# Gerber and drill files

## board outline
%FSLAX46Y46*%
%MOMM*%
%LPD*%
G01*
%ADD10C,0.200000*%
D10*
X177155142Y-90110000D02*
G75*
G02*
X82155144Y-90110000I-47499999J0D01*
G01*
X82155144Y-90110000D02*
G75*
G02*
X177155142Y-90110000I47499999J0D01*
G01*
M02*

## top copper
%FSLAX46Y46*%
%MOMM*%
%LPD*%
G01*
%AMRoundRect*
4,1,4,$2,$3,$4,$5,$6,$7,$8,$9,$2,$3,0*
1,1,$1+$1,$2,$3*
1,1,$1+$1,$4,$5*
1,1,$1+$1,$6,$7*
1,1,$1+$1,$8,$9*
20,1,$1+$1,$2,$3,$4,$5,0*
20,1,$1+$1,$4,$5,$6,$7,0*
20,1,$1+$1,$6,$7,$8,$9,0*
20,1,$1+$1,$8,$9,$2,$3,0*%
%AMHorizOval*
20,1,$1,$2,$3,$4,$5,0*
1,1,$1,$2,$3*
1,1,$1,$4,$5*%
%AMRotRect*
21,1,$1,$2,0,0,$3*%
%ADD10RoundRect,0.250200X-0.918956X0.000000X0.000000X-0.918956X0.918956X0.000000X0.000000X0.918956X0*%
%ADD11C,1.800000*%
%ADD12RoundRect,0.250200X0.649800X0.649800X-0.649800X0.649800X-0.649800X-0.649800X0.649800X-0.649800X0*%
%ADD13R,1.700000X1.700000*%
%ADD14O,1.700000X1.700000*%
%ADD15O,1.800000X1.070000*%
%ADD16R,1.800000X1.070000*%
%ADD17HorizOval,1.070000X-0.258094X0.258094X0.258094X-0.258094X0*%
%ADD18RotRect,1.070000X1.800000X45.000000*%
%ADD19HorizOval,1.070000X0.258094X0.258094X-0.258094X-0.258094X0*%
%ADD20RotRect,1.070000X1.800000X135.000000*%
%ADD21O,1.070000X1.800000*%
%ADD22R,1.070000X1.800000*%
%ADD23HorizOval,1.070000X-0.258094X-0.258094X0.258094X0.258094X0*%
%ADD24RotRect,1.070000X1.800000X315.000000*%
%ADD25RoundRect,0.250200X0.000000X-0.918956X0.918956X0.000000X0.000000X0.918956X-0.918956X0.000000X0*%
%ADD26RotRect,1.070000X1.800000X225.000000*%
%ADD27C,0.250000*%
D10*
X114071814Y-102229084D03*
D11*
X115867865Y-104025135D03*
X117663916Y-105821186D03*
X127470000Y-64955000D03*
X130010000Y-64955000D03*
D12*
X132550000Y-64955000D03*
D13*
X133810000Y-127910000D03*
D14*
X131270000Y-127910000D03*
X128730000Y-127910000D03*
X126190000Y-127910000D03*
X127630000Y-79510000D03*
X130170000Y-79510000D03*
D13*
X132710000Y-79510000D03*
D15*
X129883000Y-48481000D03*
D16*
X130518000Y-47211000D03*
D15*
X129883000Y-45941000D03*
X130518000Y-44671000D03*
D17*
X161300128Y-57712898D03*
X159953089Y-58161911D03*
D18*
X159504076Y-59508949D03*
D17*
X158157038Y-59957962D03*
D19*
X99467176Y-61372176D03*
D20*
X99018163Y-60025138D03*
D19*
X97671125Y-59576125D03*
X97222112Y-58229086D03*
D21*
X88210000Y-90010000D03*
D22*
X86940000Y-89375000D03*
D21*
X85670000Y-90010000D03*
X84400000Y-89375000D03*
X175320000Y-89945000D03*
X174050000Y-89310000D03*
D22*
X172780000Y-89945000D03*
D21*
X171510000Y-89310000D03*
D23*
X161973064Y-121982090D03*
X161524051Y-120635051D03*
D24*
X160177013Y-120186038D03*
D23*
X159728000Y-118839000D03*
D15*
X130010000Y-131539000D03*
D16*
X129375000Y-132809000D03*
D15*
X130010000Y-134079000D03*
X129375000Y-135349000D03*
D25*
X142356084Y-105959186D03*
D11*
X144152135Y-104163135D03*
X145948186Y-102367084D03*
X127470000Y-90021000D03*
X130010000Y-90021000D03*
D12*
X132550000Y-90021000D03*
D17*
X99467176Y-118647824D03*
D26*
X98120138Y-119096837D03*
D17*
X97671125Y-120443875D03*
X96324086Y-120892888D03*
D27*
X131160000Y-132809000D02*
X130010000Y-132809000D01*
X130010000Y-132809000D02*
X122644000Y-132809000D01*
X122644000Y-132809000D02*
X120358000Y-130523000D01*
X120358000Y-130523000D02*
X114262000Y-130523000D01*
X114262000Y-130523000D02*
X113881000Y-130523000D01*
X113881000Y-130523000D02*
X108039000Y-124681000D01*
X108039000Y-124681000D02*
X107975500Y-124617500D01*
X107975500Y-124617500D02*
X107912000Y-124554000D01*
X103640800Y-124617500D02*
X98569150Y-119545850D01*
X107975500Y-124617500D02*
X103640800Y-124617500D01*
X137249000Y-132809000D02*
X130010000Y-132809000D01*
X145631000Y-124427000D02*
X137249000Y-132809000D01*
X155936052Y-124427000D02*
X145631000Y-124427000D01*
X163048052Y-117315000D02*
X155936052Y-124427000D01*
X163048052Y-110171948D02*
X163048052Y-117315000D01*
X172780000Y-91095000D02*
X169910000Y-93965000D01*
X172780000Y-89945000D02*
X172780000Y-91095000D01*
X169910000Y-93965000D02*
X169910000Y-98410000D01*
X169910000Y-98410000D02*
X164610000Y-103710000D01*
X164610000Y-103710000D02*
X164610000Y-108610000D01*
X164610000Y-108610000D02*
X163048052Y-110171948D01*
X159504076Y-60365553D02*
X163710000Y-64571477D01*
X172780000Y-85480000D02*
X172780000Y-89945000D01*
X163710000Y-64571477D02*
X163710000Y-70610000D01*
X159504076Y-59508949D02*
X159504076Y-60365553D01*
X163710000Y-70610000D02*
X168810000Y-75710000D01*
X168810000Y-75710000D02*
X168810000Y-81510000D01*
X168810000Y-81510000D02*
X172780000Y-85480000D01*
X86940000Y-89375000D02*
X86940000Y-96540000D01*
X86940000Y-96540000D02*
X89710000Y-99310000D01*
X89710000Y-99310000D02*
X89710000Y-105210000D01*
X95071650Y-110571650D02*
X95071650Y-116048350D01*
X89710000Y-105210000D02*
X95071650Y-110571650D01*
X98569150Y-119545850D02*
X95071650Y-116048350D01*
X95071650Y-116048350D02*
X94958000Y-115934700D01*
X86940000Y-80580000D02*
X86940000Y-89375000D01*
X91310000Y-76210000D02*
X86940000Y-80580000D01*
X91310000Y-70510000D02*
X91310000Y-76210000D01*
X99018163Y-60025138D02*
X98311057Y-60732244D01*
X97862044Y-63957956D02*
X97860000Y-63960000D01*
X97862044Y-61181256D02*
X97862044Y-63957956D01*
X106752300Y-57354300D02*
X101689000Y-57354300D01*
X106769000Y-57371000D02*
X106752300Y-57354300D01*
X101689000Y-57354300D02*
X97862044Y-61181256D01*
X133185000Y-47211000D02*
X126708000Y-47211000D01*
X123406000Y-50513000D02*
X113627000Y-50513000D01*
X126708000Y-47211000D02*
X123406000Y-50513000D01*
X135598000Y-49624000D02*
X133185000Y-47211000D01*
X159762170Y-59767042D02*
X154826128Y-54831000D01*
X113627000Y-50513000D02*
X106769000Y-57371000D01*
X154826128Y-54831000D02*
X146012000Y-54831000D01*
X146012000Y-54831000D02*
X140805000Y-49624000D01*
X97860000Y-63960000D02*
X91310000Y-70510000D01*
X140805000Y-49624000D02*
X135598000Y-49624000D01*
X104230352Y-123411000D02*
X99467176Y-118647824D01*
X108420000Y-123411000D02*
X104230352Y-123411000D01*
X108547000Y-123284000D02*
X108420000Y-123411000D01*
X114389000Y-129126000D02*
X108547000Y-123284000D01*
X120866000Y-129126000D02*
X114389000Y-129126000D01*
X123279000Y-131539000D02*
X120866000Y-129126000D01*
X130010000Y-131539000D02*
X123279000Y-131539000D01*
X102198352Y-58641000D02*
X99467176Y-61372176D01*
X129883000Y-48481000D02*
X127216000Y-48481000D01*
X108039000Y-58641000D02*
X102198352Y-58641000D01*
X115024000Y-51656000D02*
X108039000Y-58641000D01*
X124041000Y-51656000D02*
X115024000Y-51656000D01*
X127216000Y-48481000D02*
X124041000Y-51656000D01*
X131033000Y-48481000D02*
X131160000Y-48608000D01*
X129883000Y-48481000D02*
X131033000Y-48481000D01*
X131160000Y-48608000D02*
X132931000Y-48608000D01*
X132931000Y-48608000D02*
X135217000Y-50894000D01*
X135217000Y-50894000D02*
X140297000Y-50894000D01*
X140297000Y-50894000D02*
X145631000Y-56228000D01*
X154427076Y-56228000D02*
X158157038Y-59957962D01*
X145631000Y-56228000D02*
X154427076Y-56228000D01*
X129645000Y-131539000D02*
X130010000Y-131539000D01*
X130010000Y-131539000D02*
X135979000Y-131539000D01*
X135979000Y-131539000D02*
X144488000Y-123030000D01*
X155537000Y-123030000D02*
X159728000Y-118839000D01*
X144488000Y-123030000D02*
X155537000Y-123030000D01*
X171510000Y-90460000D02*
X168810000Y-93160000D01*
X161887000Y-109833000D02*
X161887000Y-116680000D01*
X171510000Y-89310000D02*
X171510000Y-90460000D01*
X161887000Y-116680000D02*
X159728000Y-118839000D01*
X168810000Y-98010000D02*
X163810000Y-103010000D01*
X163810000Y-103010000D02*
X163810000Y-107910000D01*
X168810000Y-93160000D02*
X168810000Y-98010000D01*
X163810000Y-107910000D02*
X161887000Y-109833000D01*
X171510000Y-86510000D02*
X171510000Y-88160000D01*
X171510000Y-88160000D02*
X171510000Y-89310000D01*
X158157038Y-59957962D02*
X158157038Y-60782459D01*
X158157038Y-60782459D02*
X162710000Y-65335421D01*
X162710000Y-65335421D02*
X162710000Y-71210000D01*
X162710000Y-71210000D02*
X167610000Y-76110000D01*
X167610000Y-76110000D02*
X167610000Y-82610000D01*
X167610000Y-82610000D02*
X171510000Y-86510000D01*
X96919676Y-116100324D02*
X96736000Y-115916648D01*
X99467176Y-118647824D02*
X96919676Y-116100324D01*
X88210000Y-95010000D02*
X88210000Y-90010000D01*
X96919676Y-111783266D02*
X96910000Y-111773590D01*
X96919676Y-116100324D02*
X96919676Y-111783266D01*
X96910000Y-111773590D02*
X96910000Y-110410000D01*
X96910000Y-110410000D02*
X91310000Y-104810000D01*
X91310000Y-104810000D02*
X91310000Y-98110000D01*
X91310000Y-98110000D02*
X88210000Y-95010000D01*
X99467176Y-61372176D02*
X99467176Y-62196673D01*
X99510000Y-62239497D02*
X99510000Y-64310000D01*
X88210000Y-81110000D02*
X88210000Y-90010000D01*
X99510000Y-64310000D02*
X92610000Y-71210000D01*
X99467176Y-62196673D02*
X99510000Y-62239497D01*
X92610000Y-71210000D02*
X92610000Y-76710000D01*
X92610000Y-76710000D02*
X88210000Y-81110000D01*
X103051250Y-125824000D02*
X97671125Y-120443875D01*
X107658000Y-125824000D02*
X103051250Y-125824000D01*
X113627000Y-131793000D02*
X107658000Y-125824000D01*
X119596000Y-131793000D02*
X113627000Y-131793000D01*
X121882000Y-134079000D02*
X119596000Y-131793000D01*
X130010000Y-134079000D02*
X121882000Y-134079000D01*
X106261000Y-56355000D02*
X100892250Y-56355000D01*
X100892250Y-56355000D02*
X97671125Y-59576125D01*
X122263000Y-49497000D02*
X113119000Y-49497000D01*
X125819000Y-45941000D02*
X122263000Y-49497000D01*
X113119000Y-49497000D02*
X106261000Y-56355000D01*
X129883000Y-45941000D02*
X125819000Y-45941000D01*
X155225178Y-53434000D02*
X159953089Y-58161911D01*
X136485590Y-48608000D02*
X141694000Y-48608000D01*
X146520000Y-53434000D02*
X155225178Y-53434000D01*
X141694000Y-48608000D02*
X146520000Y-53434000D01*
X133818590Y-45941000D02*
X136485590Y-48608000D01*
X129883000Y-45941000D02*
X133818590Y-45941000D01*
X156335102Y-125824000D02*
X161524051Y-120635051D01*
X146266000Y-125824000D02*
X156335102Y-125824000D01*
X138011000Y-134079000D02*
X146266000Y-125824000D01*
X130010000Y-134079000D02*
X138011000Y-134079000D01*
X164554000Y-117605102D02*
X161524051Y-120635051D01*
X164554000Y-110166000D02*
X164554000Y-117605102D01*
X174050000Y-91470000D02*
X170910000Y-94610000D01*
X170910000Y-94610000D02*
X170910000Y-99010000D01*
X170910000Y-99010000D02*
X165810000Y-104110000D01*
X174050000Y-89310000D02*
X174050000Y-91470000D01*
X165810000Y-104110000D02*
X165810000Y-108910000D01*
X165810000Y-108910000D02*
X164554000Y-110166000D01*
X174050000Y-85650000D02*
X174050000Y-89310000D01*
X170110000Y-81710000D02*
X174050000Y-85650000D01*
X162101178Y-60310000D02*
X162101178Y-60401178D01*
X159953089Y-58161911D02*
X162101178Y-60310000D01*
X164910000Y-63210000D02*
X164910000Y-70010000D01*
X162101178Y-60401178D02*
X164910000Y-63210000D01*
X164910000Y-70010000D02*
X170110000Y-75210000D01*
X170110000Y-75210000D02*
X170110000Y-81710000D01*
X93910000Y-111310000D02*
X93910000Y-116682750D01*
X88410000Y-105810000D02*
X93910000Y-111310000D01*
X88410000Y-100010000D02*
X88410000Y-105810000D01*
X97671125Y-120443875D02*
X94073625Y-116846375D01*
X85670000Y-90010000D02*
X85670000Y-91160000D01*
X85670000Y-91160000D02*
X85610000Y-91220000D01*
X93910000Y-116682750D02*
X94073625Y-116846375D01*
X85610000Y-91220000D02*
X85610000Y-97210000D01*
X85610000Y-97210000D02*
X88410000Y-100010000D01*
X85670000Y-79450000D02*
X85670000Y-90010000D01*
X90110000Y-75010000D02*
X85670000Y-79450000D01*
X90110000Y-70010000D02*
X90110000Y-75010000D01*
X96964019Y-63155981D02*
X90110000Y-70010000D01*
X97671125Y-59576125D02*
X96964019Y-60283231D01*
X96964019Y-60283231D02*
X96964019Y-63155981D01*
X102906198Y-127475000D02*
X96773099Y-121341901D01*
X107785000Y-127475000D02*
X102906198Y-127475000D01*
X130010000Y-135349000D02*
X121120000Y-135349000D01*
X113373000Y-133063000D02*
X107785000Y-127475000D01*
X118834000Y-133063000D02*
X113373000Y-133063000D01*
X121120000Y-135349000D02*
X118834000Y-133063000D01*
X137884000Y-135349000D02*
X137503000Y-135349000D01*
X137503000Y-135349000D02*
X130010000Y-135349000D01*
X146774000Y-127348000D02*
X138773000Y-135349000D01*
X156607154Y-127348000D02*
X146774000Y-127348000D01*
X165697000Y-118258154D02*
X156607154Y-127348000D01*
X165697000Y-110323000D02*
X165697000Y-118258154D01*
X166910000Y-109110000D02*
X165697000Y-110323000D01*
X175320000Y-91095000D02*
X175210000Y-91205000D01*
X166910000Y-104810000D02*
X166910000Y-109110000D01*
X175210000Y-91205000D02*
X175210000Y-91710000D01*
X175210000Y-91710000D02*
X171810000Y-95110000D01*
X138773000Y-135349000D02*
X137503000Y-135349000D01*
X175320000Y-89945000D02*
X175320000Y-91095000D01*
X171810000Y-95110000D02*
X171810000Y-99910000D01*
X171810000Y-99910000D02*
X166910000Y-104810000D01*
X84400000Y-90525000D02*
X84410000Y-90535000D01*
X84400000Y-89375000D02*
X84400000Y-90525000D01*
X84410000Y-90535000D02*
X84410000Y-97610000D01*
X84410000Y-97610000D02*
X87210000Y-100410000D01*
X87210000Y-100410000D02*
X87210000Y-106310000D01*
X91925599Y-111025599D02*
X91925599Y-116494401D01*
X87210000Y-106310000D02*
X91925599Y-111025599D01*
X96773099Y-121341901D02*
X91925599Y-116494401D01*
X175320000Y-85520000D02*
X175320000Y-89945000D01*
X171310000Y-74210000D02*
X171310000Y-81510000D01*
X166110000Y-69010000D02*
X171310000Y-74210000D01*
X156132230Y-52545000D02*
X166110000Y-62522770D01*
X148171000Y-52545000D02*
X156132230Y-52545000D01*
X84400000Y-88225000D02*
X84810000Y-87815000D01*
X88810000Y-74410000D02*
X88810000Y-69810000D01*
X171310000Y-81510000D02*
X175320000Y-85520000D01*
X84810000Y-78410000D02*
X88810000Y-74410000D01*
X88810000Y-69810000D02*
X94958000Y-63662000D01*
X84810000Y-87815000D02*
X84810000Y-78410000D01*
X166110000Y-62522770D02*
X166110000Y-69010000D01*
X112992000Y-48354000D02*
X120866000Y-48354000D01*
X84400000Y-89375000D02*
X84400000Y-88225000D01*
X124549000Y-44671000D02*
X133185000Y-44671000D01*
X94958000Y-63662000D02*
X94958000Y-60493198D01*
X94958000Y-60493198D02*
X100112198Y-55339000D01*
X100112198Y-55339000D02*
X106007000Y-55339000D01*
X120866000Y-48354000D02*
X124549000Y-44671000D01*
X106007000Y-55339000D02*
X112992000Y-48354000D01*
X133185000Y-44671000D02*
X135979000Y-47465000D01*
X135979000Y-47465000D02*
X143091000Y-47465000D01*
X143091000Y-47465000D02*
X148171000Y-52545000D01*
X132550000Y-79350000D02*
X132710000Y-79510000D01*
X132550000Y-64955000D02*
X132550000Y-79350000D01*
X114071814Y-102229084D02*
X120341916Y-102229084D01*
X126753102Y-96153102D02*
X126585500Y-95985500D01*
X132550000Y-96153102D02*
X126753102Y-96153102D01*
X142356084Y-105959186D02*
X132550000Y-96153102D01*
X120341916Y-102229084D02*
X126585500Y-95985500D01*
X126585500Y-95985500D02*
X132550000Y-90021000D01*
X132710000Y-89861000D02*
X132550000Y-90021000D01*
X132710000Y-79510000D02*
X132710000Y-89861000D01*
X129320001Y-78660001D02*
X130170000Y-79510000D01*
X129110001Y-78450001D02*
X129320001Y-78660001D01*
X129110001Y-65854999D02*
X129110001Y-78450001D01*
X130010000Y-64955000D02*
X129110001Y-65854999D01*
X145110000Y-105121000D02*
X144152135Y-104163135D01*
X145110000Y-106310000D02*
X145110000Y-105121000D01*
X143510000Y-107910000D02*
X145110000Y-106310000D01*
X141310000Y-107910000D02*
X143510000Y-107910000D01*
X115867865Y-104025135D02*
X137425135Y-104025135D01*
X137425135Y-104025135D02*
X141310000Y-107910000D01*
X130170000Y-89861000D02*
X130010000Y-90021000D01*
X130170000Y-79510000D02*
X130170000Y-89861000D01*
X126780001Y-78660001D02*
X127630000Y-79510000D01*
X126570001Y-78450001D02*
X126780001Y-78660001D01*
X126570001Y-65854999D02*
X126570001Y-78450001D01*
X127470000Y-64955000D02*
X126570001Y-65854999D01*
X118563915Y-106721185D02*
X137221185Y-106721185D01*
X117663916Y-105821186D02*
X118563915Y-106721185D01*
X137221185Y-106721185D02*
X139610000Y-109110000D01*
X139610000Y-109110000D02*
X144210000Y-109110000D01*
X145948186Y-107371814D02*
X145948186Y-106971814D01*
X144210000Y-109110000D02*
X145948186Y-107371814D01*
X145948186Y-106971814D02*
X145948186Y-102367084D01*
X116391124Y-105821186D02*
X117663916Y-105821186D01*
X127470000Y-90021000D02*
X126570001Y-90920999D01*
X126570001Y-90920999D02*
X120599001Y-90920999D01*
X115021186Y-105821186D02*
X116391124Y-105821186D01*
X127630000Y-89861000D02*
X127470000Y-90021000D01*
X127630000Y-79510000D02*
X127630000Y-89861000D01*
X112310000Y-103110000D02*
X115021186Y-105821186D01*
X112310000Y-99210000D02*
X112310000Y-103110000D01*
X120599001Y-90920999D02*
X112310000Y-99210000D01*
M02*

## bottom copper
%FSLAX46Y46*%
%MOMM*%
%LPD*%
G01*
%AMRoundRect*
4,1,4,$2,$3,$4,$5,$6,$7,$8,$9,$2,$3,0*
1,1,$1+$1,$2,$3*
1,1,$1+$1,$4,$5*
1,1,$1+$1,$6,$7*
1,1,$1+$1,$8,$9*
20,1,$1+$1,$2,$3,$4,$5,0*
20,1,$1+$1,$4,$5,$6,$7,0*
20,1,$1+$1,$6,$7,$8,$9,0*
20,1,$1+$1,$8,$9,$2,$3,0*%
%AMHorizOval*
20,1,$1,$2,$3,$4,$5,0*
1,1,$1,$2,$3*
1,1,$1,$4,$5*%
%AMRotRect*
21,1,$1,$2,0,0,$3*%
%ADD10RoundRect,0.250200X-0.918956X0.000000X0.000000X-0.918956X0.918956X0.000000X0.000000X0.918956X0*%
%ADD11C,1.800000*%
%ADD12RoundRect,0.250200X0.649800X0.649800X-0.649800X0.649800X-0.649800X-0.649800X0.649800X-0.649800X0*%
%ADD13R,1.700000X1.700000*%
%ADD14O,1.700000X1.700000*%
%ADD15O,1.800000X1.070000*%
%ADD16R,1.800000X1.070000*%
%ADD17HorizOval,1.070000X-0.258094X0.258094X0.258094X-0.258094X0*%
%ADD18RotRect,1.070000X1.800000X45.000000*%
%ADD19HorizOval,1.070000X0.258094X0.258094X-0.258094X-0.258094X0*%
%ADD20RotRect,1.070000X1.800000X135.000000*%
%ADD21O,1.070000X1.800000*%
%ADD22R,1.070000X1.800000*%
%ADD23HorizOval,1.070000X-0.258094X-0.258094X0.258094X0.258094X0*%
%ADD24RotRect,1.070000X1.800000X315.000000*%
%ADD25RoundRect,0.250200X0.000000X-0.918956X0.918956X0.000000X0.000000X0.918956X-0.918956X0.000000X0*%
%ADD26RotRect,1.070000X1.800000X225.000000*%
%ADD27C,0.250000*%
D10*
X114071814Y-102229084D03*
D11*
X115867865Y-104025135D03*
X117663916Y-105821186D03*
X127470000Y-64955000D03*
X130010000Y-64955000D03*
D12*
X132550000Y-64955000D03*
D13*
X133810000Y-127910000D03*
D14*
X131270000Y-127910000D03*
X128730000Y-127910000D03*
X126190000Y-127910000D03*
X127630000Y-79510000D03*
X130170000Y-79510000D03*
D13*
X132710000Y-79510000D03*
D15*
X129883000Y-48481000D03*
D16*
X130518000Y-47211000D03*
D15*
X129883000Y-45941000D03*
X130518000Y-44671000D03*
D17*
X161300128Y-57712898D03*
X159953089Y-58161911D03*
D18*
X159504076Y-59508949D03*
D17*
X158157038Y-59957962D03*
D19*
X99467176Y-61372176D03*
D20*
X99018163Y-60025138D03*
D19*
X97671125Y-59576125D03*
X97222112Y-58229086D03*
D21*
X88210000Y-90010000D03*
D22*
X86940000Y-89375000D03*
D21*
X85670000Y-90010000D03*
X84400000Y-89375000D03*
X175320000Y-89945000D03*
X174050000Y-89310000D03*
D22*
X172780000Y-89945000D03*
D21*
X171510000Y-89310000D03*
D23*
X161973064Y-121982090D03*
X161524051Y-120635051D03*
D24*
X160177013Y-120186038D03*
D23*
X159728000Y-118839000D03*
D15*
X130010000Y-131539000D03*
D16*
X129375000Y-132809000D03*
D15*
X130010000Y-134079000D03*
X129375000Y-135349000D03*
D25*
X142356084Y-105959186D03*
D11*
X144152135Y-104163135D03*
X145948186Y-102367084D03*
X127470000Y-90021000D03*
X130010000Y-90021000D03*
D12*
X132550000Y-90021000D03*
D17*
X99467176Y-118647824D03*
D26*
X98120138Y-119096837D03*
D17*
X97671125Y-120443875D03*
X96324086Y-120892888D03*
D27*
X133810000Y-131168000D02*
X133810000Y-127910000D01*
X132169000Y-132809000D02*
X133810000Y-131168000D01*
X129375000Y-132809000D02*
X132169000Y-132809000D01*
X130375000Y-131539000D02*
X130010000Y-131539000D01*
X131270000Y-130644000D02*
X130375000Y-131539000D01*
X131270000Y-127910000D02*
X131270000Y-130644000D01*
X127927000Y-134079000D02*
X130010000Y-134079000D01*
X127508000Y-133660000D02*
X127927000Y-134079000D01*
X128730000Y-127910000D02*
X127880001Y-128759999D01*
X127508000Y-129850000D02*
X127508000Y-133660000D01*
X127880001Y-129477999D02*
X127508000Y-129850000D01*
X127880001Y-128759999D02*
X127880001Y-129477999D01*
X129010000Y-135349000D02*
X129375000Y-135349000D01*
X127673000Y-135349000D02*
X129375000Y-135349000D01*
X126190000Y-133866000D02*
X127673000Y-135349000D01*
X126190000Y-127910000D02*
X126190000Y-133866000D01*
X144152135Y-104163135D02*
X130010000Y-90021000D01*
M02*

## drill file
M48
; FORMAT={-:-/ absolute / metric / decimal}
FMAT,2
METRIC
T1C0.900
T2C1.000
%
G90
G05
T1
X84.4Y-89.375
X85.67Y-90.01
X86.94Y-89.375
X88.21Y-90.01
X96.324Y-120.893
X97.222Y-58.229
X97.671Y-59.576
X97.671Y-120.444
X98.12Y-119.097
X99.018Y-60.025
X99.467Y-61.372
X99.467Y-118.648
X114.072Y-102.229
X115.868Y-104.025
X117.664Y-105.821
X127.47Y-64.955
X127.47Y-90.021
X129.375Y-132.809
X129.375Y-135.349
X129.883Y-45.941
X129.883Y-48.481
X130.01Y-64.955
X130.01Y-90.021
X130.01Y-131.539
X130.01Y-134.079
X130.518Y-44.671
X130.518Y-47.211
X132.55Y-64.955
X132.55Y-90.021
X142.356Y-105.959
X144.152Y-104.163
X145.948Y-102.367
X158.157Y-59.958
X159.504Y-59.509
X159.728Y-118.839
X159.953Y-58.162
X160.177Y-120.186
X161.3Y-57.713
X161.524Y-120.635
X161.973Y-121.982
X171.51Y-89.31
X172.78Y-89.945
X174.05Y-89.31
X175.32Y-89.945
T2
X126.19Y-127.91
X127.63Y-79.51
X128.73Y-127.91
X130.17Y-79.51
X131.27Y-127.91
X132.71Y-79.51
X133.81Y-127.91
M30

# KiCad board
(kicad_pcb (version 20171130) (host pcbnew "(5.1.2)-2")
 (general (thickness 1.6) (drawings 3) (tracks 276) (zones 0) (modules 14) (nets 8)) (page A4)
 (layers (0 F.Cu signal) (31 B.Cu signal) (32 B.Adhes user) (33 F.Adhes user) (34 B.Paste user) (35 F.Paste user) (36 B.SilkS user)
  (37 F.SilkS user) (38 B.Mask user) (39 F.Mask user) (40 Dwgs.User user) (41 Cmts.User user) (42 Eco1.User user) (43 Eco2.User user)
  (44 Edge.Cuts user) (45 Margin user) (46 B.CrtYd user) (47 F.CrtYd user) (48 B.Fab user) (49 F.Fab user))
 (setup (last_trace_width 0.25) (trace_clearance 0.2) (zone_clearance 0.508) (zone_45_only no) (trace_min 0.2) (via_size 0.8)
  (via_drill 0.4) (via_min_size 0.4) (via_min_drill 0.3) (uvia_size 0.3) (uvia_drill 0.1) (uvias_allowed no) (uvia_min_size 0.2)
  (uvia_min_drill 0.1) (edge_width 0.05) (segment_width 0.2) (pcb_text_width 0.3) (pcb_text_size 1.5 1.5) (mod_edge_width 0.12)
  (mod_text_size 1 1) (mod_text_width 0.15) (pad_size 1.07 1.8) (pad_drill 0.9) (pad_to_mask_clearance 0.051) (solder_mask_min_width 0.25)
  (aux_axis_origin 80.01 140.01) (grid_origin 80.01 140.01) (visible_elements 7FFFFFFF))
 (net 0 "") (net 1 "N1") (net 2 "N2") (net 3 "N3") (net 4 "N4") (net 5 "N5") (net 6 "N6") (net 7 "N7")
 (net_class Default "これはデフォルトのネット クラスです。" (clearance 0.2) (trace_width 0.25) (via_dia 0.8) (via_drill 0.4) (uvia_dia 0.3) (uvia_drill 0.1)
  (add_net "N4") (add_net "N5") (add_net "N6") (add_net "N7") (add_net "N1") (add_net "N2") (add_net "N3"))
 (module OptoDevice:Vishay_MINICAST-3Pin (layer F.Cu) (at 115.867865 104.025135 315)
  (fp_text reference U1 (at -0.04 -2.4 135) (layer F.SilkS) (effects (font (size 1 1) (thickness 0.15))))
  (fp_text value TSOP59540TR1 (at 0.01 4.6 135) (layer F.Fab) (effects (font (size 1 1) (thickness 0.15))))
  (pad 1 thru_hole roundrect (at -2.54 0 315) (size 1.8 1.8) (drill 0.9) (layers *.Cu *.Mask) (roundrect_rratio 0.139) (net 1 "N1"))
  (pad 2 thru_hole circle (at 0 0 315) (size 1.8 1.8) (drill 0.9) (layers *.Cu *.Mask) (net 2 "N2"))
  (pad 3 thru_hole circle (at 2.54 0 315) (size 1.8 1.8) (drill 0.9) (layers *.Cu *.Mask) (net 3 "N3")))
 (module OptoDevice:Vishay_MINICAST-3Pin (layer F.Cu) (at 130.01 64.955 180)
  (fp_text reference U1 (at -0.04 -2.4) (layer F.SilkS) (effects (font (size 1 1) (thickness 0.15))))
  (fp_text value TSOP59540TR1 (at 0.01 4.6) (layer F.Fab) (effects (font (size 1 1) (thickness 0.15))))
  (pad 3 thru_hole circle (at 2.54 0 180) (size 1.8 1.8) (drill 0.9) (layers *.Cu *.Mask) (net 3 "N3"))
  (pad 2 thru_hole circle (at 0 0 180) (size 1.8 1.8) (drill 0.9) (layers *.Cu *.Mask) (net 2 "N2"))
  (pad 1 thru_hole roundrect (at -2.54 0 180) (size 1.8 1.8) (drill 0.9) (layers *.Cu *.Mask) (roundrect_rratio 0.139) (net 1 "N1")))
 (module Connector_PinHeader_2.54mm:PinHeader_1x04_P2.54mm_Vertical (layer B.Cu) (at 133.81 127.91 90)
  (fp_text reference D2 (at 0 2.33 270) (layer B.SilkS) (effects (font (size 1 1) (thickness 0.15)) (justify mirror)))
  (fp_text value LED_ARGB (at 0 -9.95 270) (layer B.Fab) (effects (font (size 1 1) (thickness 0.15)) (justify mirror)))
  (pad 1 thru_hole rect (at 0 0 90) (size 1.7 1.7) (drill 1) (layers *.Cu *.Mask) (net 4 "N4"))
  (pad 2 thru_hole oval (at 0 -2.54 90) (size 1.7 1.7) (drill 1) (layers *.Cu *.Mask) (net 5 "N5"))
  (pad 3 thru_hole oval (at 0 -5.08 90) (size 1.7 1.7) (drill 1) (layers *.Cu *.Mask) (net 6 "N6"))
  (pad 4 thru_hole oval (at 0 -7.62 90) (size 1.7 1.7) (drill 1) (layers *.Cu *.Mask) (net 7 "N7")))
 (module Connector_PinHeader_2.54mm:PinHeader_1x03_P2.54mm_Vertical (layer B.Cu) (at 132.71 79.51 90)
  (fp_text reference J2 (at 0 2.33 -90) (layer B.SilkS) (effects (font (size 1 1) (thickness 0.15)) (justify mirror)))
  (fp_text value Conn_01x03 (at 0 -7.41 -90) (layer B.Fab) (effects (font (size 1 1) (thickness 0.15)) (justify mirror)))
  (pad 3 thru_hole oval (at 0 -5.08 90) (size 1.7 1.7) (drill 1) (layers *.Cu *.Mask) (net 3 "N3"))
  (pad 2 thru_hole oval (at 0 -2.54 90) (size 1.7 1.7) (drill 1) (layers *.Cu *.Mask) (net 2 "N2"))
  (pad 1 thru_hole rect (at 0 0 90) (size 1.7 1.7) (drill 1) (layers *.Cu *.Mask) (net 1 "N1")))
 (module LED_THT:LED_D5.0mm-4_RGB (layer F.Cu) (at 129.883 48.481 90)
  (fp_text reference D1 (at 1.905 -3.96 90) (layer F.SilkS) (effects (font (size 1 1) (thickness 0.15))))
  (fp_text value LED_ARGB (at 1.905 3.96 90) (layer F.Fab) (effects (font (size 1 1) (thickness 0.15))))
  (pad 1 thru_hole oval (at 0 0 90) (size 1.07 1.8) (drill 0.9) (layers *.Cu *.Mask) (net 5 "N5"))
  (pad 2 thru_hole rect (at 1.27 0.635 90) (size 1.07 1.8) (drill 0.9) (layers *.Cu *.Mask) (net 4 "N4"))
  (pad 3 thru_hole oval (at 2.54 0 90) (size 1.07 1.8) (drill 0.9) (layers *.Cu *.Mask) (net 6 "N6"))
  (pad 4 thru_hole oval (at 3.81 0.635 90) (size 1.07 1.8) (drill 0.9) (layers *.Cu *.Mask) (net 7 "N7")))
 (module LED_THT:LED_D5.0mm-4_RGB (layer F.Cu) (at 158.157038 59.957962 45)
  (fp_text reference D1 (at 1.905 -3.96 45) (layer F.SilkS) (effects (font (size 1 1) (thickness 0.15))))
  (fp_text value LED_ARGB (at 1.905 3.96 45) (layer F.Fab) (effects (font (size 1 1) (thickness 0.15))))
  (pad 4 thru_hole oval (at 3.81 0.635 45) (size 1.07 1.8) (drill 0.9) (layers *.Cu *.Mask) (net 7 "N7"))
  (pad 3 thru_hole oval (at 2.54 0 45) (size 1.07 1.8) (drill 0.9) (layers *.Cu *.Mask) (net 6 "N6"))
  (pad 2 thru_hole rect (at 1.27 0.635 45) (size 1.07 1.8) (drill 0.9) (layers *.Cu *.Mask) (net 4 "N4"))
  (pad 1 thru_hole oval (at 0 0 45) (size 1.07 1.8) (drill 0.9) (layers *.Cu *.Mask) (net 5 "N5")))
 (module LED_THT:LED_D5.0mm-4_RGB (layer F.Cu) (at 99.467176 61.372176 135)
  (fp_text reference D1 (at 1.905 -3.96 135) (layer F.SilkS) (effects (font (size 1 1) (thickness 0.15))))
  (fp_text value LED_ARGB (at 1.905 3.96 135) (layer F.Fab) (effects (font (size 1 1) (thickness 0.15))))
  (pad 1 thru_hole oval (at 0 0 135) (size 1.07 1.8) (drill 0.9) (layers *.Cu *.Mask) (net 5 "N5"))
  (pad 2 thru_hole rect (at 1.27 0.635 135) (size 1.07 1.8) (drill 0.9) (layers *.Cu *.Mask) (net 4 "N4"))
  (pad 3 thru_hole oval (at 2.54 0 135) (size 1.07 1.8) (drill 0.9) (layers *.Cu *.Mask) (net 6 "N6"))
  (pad 4 thru_hole oval (at 3.81 0.635 135) (size 1.07 1.8) (drill 0.9) (layers *.Cu *.Mask) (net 7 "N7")))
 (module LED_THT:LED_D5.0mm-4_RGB (layer F.Cu) (at 88.21 90.01 180)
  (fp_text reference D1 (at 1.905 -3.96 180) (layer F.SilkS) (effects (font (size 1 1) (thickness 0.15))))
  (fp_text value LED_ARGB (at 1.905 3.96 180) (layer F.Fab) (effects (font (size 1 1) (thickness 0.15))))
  (pad 1 thru_hole oval (at 0 0 180) (size 1.07 1.8) (drill 0.9) (layers *.Cu *.Mask) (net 5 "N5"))
  (pad 2 thru_hole rect (at 1.27 0.635 180) (size 1.07 1.8) (drill 0.9) (layers *.Cu *.Mask) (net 4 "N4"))
  (pad 3 thru_hole oval (at 2.54 0 180) (size 1.07 1.8) (drill 0.9) (layers *.Cu *.Mask) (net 6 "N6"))
  (pad 4 thru_hole oval (at 3.81 0.635 180) (size 1.07 1.8) (drill 0.9) (layers *.Cu *.Mask) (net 7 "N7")))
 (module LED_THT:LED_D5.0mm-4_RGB (layer F.Cu) (at 171.51 89.31)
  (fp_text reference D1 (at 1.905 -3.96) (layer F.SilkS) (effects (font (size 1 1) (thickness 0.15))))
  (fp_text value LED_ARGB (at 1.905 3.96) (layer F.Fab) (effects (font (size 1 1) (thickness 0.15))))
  (pad 4 thru_hole oval (at 3.81 0.635) (size 1.07 1.8) (drill 0.9) (layers *.Cu *.Mask) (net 7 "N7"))
  (pad 3 thru_hole oval (at 2.54 0) (size 1.07 1.8) (drill 0.9) (layers *.Cu *.Mask) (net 6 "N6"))
  (pad 2 thru_hole rect (at 1.27 0.635) (size 1.07 1.8) (drill 0.9) (layers *.Cu *.Mask) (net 4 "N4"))
  (pad 1 thru_hole oval (at 0 0) (size 1.07 1.8) (drill 0.9) (layers *.Cu *.Mask) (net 5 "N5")))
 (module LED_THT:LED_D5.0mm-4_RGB (layer F.Cu) (at 159.728 118.839 315)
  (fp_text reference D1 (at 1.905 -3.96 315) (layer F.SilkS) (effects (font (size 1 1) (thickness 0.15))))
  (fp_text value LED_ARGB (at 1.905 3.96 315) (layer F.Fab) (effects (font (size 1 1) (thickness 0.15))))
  (pad 4 thru_hole oval (at 3.81 0.635 315) (size 1.07 1.8) (drill 0.9) (layers *.Cu *.Mask) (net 7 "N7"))
  (pad 3 thru_hole oval (at 2.54 0 315) (size 1.07 1.8) (drill 0.9) (layers *.Cu *.Mask) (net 6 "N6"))
  (pad 2 thru_hole rect (at 1.27 0.635 315) (size 1.07 1.8) (drill 0.9) (layers *.Cu *.Mask) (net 4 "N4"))
  (pad 1 thru_hole oval (at 0 0 315) (size 1.07 1.8) (drill 0.9) (layers *.Cu *.Mask) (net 5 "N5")))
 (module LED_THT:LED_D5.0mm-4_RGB (layer F.Cu) (at 130.01 131.539 270)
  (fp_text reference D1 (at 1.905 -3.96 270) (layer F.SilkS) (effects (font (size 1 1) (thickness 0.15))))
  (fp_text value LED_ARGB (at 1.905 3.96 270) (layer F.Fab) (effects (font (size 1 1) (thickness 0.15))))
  (pad 1 thru_hole oval (at 0 0 270) (size 1.07 1.8) (drill 0.9) (layers *.Cu *.Mask) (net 5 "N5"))
  (pad 2 thru_hole rect (at 1.27 0.635 270) (size 1.07 1.8) (drill 0.9) (layers *.Cu *.Mask) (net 4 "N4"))
  (pad 3 thru_hole oval (at 2.54 0 270) (size 1.07 1.8) (drill 0.9) (layers *.Cu *.Mask) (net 6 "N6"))
  (pad 4 thru_hole oval (at 3.81 0.635 270) (size 1.07 1.8) (drill 0.9) (layers *.Cu *.Mask) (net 7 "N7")))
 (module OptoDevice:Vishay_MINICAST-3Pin (layer F.Cu) (at 144.152135 104.163135 45)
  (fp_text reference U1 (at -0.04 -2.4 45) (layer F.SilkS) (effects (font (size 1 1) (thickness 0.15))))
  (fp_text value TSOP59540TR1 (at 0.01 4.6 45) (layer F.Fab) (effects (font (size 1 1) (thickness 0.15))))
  (pad 1 thru_hole roundrect (at -2.54 0 45) (size 1.8 1.8) (drill 0.9) (layers *.Cu *.Mask) (roundrect_rratio 0.139) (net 1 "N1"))
  (pad 2 thru_hole circle (at 0 0 45) (size 1.8 1.8) (drill 0.9) (layers *.Cu *.Mask) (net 2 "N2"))
  (pad 3 thru_hole circle (at 2.54 0 45) (size 1.8 1.8) (drill 0.9) (layers *.Cu *.Mask) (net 3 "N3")))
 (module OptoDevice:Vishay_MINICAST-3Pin (layer F.Cu) (at 130.01 90.021 180)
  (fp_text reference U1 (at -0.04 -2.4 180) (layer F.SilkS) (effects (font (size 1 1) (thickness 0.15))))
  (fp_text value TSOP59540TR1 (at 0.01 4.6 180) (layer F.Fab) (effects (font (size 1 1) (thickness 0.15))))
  (pad 3 thru_hole circle (at 2.54 0 180) (size 1.8 1.8) (drill 0.9) (layers *.Cu *.Mask) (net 3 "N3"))
  (pad 2 thru_hole circle (at 0 0 180) (size 1.8 1.8) (drill 0.9) (layers *.Cu *.Mask) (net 2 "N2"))
  (pad 1 thru_hole roundrect (at -2.54 0 180) (size 1.8 1.8) (drill 0.9) (layers *.Cu *.Mask) (roundrect_rratio 0.139) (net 1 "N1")))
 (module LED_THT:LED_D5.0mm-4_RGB (layer F.Cu) (at 99.467176 118.647824 225)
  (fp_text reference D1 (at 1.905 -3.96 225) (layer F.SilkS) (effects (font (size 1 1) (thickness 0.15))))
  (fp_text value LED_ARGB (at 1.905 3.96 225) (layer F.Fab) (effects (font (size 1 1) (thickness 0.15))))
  (pad 1 thru_hole oval (at 0 0 225) (size 1.07 1.8) (drill 0.9) (layers *.Cu *.Mask) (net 5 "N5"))
  (pad 2 thru_hole rect (at 1.27 0.635 225) (size 1.07 1.8) (drill 0.9) (layers *.Cu *.Mask) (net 4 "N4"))
  (pad 3 thru_hole oval (at 2.54 0 225) (size 1.07 1.8) (drill 0.9) (layers *.Cu *.Mask) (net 6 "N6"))
  (pad 4 thru_hole oval (at 3.81 0.635 225) (size 1.07 1.8) (drill 0.9) (layers *.Cu *.Mask) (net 7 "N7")))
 (gr_circle (center 129.655143 90.11) (end 177.155142 90.11) (layer Edge.Cuts) (width 0.2))
 (segment (start 131.16 132.809) (end 130.01 132.809) (width 0.25) (layer F.Cu) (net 4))
 (segment (start 130.01 132.809) (end 122.644 132.809) (width 0.25) (layer F.Cu) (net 4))
 (segment (start 122.644 132.809) (end 120.358 130.523) (width 0.25) (layer F.Cu) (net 4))
 (segment (start 120.358 130.523) (end 114.262 130.523) (width 0.25) (layer F.Cu) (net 4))
 (segment (start 114.262 130.523) (end 113.881 130.523) (width 0.25) (layer F.Cu) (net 4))
 (segment (start 113.881 130.523) (end 108.039 124.681) (width 0.25) (layer F.Cu) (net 4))
 (segment (start 108.039 124.681) (end 107.9755 124.6175) (width 0.25) (layer F.Cu) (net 4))
 (segment (start 107.9755 124.6175) (end 107.912 124.554) (width 0.25) (layer F.Cu) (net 4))
 (segment (start 103.6408 124.6175) (end 98.56915 119.54585) (width 0.25) (layer F.Cu) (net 4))
 (segment (start 107.9755 124.6175) (end 103.6408 124.6175) (width 0.25) (layer F.Cu) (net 4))
 (segment (start 133.81 131.168) (end 133.81 127.91) (width 0.25) (layer B.Cu) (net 4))
 (segment (start 132.169 132.809) (end 133.81 131.168) (width 0.25) (layer B.Cu) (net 4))
 (segment (start 129.375 132.809) (end 132.169 132.809) (width 0.25) (layer B.Cu) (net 4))
 (segment (start 137.249 132.809) (end 130.01 132.809) (width 0.25) (layer F.Cu) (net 4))
 (segment (start 145.631 124.427) (end 137.249 132.809) (width 0.25) (layer F.Cu) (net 4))
 (segment (start 155.936052 124.427) (end 145.631 124.427) (width 0.25) (layer F.Cu) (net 4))
 (segment (start 163.048052 117.315) (end 155.936052 124.427) (width 0.25) (layer F.Cu) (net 4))
 (segment (start 163.048052 110.171948) (end 163.048052 117.315) (width 0.25) (layer F.Cu) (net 4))
 (segment (start 172.78 91.095) (end 169.91 93.965) (width 0.25) (layer F.Cu) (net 4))
 (segment (start 172.78 89.945) (end 172.78 91.095) (width 0.25) (layer F.Cu) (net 4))
 (segment (start 169.91 93.965) (end 169.91 98.41) (width 0.25) (layer F.Cu) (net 4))
 (segment (start 169.91 98.41) (end 164.61 103.71) (width 0.25) (layer F.Cu) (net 4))
 (segment (start 164.61 103.71) (end 164.61 108.61) (width 0.25) (layer F.Cu) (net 4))
 (segment (start 164.61 108.61) (end 163.048052 110.171948) (width 0.25) (layer F.Cu) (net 4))
 (segment (start 159.504076 60.365553) (end 163.71 64.571477) (width 0.25) (layer F.Cu) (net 4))
 (segment (start 172.78 85.48) (end 172.78 89.945) (width 0.25) (layer F.Cu) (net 4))
 (segment (start 163.71 64.571477) (end 163.71 70.61) (width 0.25) (layer F.Cu) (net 4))
 (segment (start 159.504076 59.508949) (end 159.504076 60.365553) (width 0.25) (layer F.Cu) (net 4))
 (segment (start 163.71 70.61) (end 168.81 75.71) (width 0.25) (layer F.Cu) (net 4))
 (segment (start 168.81 75.71) (end 168.81 81.51) (width 0.25) (layer F.Cu) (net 4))
 (segment (start 168.81 81.51) (end 172.78 85.48) (width 0.25) (layer F.Cu) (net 4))
 (segment (start 86.94 89.375) (end 86.94 96.54) (width 0.25) (layer F.Cu) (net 4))
 (segment (start 86.94 96.54) (end 89.71 99.31) (width 0.25) (layer F.Cu) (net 4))
 (segment (start 89.71 99.31) (end 89.71 105.21) (width 0.25) (layer F.Cu) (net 4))
 (segment (start 95.07165 110.57165) (end 95.07165 116.04835) (width 0.25) (layer F.Cu) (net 4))
 (segment (start 89.71 105.21) (end 95.07165 110.57165) (width 0.25) (layer F.Cu) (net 4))
 (segment (start 98.56915 119.54585) (end 95.07165 116.04835) (width 0.25) (layer F.Cu) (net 4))
 (segment (start 95.07165 116.04835) (end 94.958 115.9347) (width 0.25) (layer F.Cu) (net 4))
 (segment (start 86.94 80.58) (end 86.94 89.375) (width 0.25) (layer F.Cu) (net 4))
 (segment (start 91.31 76.21) (end 86.94 80.58) (width 0.25) (layer F.Cu) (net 4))
 (segment (start 91.31 70.51) (end 91.31 76.21) (width 0.25) (layer F.Cu) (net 4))
 (segment (start 99.018163 60.025138) (end 98.311057 60.732244) (width 0.25) (layer F.Cu) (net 4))
 (segment (start 97.862044 63.957956) (end 97.86 63.96) (width 0.25) (layer F.Cu) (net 4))
 (segment (start 97.862044 61.181256) (end 97.862044 63.957956) (width 0.25) (layer F.Cu) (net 4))
 (segment (start 106.7523 57.3543) (end 101.689 57.3543) (width 0.25) (layer F.Cu) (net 4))
 (segment (start 106.769 57.371) (end 106.7523 57.3543) (width 0.25) (layer F.Cu) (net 4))
 (segment (start 101.689 57.3543) (end 97.862044 61.181256) (width 0.25) (layer F.Cu) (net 4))
 (segment (start 133.185 47.211) (end 126.708 47.211) (width 0.25) (layer F.Cu) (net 4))
 (segment (start 123.406 50.513) (end 113.627 50.513) (width 0.25) (layer F.Cu) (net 4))
 (segment (start 126.708 47.211) (end 123.406 50.513) (width 0.25) (layer F.Cu) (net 4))
 (segment (start 135.598 49.624) (end 133.185 47.211) (width 0.25) (layer F.Cu) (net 4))
 (segment (start 159.76217 59.767042) (end 154.826128 54.831) (width 0.25) (layer F.Cu) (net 4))
 (segment (start 113.627 50.513) (end 106.769 57.371) (width 0.25) (layer F.Cu) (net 4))
 (segment (start 154.826128 54.831) (end 146.012 54.831) (width 0.25) (layer F.Cu) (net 4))
 (segment (start 146.012 54.831) (end 140.805 49.624) (width 0.25) (layer F.Cu) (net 4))
 (segment (start 97.86 63.96) (end 91.31 70.51) (width 0.25) (layer F.Cu) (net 4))
 (segment (start 140.805 49.624) (end 135.598 49.624) (width 0.25) (layer F.Cu) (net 4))
 (segment (start 104.230352 123.411) (end 99.467176 118.647824) (width 0.25) (layer F.Cu) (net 5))
 (segment (start 108.42 123.411) (end 104.230352 123.411) (width 0.25) (layer F.Cu) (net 5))
 (segment (start 108.547 123.284) (end 108.42 123.411) (width 0.25) (layer F.Cu) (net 5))
 (segment (start 114.389 129.126) (end 108.547 123.284) (width 0.25) (layer F.Cu) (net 5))
 (segment (start 120.866 129.126) (end 114.389 129.126) (width 0.25) (layer F.Cu) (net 5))
 (segment (start 123.279 131.539) (end 120.866 129.126) (width 0.25) (layer F.Cu) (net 5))
 (segment (start 130.01 131.539) (end 123.279 131.539) (width 0.25) (layer F.Cu) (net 5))
 (segment (start 102.198352 58.641) (end 99.467176 61.372176) (width 0.25) (layer F.Cu) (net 5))
 (segment (start 129.883 48.481) (end 127.216 48.481) (width 0.25) (layer F.Cu) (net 5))
 (segment (start 108.039 58.641) (end 102.198352 58.641) (width 0.25) (layer F.Cu) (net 5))
 (segment (start 115.024 51.656) (end 108.039 58.641) (width 0.25) (layer F.Cu) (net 5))
 (segment (start 124.041 51.656) (end 115.024 51.656) (width 0.25) (layer F.Cu) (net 5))
 (segment (start 127.216 48.481) (end 124.041 51.656) (width 0.25) (layer F.Cu) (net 5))
 (segment (start 131.033 48.481) (end 131.16 48.608) (width 0.25) (layer F.Cu) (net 5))
 (segment (start 129.883 48.481) (end 131.033 48.481) (width 0.25) (layer F.Cu) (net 5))
 (segment (start 131.16 48.608) (end 132.931 48.608) (width 0.25) (layer F.Cu) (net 5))
 (segment (start 132.931 48.608) (end 135.217 50.894) (width 0.25) (layer F.Cu) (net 5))
 (segment (start 135.217 50.894) (end 140.297 50.894) (width 0.25) (layer F.Cu) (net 5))
 (segment (start 140.297 50.894) (end 145.631 56.228) (width 0.25) (layer F.Cu) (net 5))
 (segment (start 154.427076 56.228) (end 158.157038 59.957962) (width 0.25) (layer F.Cu) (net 5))
 (segment (start 145.631 56.228) (end 154.427076 56.228) (width 0.25) (layer F.Cu) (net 5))
 (segment (start 129.645 131.539) (end 130.01 131.539) (width 0.25) (layer F.Cu) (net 5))
 (segment (start 130.01 131.539) (end 135.979 131.539) (width 0.25) (layer F.Cu) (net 5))
 (segment (start 135.979 131.539) (end 144.488 123.03) (width 0.25) (layer F.Cu) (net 5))
 (segment (start 155.537 123.03) (end 159.728 118.839) (width 0.25) (layer F.Cu) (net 5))
 (segment (start 144.488 123.03) (end 155.537 123.03) (width 0.25) (layer F.Cu) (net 5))
 (segment (start 130.375 131.539) (end 130.01 131.539) (width 0.25) (layer B.Cu) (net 5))
 (segment (start 131.27 130.644) (end 130.375 131.539) (width 0.25) (layer B.Cu) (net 5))
 (segment (start 131.27 127.91) (end 131.27 130.644) (width 0.25) (layer B.Cu) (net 5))
 (segment (start 171.51 90.46) (end 168.81 93.16) (width 0.25) (layer F.Cu) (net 5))
 (segment (start 161.887 109.833) (end 161.887 116.68) (width 0.25) (layer F.Cu) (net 5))
 (segment (start 171.51 89.31) (end 171.51 90.46) (width 0.25) (layer F.Cu) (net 5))
 (segment (start 161.887 116.68) (end 159.728 118.839) (width 0.25) (layer F.Cu) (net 5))
 (segment (start 168.81 98.01) (end 163.81 103.01) (width 0.25) (layer F.Cu) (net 5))
 (segment (start 163.81 103.01) (end 163.81 107.91) (width 0.25) (layer F.Cu) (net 5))
 (segment (start 168.81 93.16) (end 168.81 98.01) (width 0.25) (layer F.Cu) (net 5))
 (segment (start 163.81 107.91) (end 161.887 109.833) (width 0.25) (layer F.Cu) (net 5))
 (segment (start 171.51 86.51) (end 171.51 88.16) (width 0.25) (layer F.Cu) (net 5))
 (segment (start 171.51 88.16) (end 171.51 89.31) (width 0.25) (layer F.Cu) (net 5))
 (segment (start 158.157038 59.957962) (end 158.157038 60.782459) (width 0.25) (layer F.Cu) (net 5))
 (segment (start 158.157038 60.782459) (end 162.71 65.335421) (width 0.25) (layer F.Cu) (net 5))
 (segment (start 162.71 65.335421) (end 162.71 71.21) (width 0.25) (layer F.Cu) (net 5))
 (segment (start 162.71 71.21) (end 167.61 76.11) (width 0.25) (layer F.Cu) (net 5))
 (segment (start 167.61 76.11) (end 167.61 82.61) (width 0.25) (layer F.Cu) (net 5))
 (segment (start 167.61 82.61) (end 171.51 86.51) (width 0.25) (layer F.Cu) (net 5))
 (segment (start 96.919676 116.100324) (end 96.736 115.916648) (width 0.25) (layer F.Cu) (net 5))
 (segment (start 99.467176 118.647824) (end 96.919676 116.100324) (width 0.25) (layer F.Cu) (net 5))
 (segment (start 88.21 95.01) (end 88.21 90.01) (width 0.25) (layer F.Cu) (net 5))
 (segment (start 96.919676 111.783266) (end 96.91 111.77359) (width 0.25) (layer F.Cu) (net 5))
 (segment (start 96.919676 116.100324) (end 96.919676 111.783266) (width 0.25) (layer F.Cu) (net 5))
 (segment (start 96.91 111.77359) (end 96.91 110.41) (width 0.25) (layer F.Cu) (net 5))
 (segment (start 96.91 110.41) (end 91.31 104.81) (width 0.25) (layer F.Cu) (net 5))
 (segment (start 91.31 104.81) (end 91.31 98.11) (width 0.25) (layer F.Cu) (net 5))
 (segment (start 91.31 98.11) (end 88.21 95.01) (width 0.25) (layer F.Cu) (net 5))
 (segment (start 99.467176 61.372176) (end 99.467176 62.196673) (width 0.25) (layer F.Cu) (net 5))
 (segment (start 99.51 62.239497) (end 99.51 64.31) (width 0.25) (layer F.Cu) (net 5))
 (segment (start 88.21 81.11) (end 88.21 90.01) (width 0.25) (layer F.Cu) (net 5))
 (segment (start 99.51 64.31) (end 92.61 71.21) (width 0.25) (layer F.Cu) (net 5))
 (segment (start 99.467176 62.196673) (end 99.51 62.239497) (width 0.25) (layer F.Cu) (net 5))
 (segment (start 92.61 71.21) (end 92.61 76.71) (width 0.25) (layer F.Cu) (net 5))
 (segment (start 92.61 76.71) (end 88.21 81.11) (width 0.25) (layer F.Cu) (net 5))
 (segment (start 103.05125 125.824) (end 97.671125 120.443875) (width 0.25) (layer F.Cu) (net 6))
 (segment (start 107.658 125.824) (end 103.05125 125.824) (width 0.25) (layer F.Cu) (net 6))
 (segment (start 113.627 131.793) (end 107.658 125.824) (width 0.25) (layer F.Cu) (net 6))
 (segment (start 119.596 131.793) (end 113.627 131.793) (width 0.25) (layer F.Cu) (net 6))
 (segment (start 121.882 134.079) (end 119.596 131.793) (width 0.25) (layer F.Cu) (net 6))
 (segment (start 130.01 134.079) (end 121.882 134.079) (width 0.25) (layer F.Cu) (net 6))
 (segment (start 106.261 56.355) (end 100.89225 56.355) (width 0.25) (layer F.Cu) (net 6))
 (segment (start 100.89225 56.355) (end 97.671125 59.576125) (width 0.25) (layer F.Cu) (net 6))
 (segment (start 122.263 49.497) (end 113.119 49.497) (width 0.25) (layer F.Cu) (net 6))
 (segment (start 125.819 45.941) (end 122.263 49.497) (width 0.25) (layer F.Cu) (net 6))
 (segment (start 113.119 49.497) (end 106.261 56.355) (width 0.25) (layer F.Cu) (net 6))
 (segment (start 129.883 45.941) (end 125.819 45.941) (width 0.25) (layer F.Cu) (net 6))
 (segment (start 155.225178 53.434) (end 159.953089 58.161911) (width 0.25) (layer F.Cu) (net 6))
 (segment (start 136.48559 48.608) (end 141.694 48.608) (width 0.25) (layer F.Cu) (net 6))
 (segment (start 146.52 53.434) (end 155.225178 53.434) (width 0.25) (layer F.Cu) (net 6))
 (segment (start 141.694 48.608) (end 146.52 53.434) (width 0.25) (layer F.Cu) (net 6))
 (segment (start 133.81859 45.941) (end 136.48559 48.608) (width 0.25) (layer F.Cu) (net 6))
 (segment (start 129.883 45.941) (end 133.81859 45.941) (width 0.25) (layer F.Cu) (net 6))
 (segment (start 156.335102 125.824) (end 161.524051 120.635051) (width 0.25) (layer F.Cu) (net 6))
 (segment (start 146.266 125.824) (end 156.335102 125.824) (width 0.25) (layer F.Cu) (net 6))
 (segment (start 138.011 134.079) (end 146.266 125.824) (width 0.25) (layer F.Cu) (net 6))
 (segment (start 130.01 134.079) (end 138.011 134.079) (width 0.25) (layer F.Cu) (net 6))
 (segment (start 127.927 134.079) (end 130.01 134.079) (width 0.25) (layer B.Cu) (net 6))
 (segment (start 127.508 133.66) (end 127.927 134.079) (width 0.25) (layer B.Cu) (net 6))
 (segment (start 128.73 127.91) (end 127.880001 128.759999) (width 0.25) (layer B.Cu) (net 6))
 (segment (start 127.508 129.85) (end 127.508 133.66) (width 0.25) (layer B.Cu) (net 6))
 (segment (start 127.880001 129.477999) (end 127.508 129.85) (width 0.25) (layer B.Cu) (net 6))
 (segment (start 127.880001 128.759999) (end 127.880001 129.477999) (width 0.25) (layer B.Cu) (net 6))
 (segment (start 164.554 117.605102) (end 161.524051 120.635051) (width 0.25) (layer F.Cu) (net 6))
 (segment (start 164.554 110.166) (end 164.554 117.605102) (width 0.25) (layer F.Cu) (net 6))
 (segment (start 174.05 91.47) (end 170.91 94.61) (width 0.25) (layer F.Cu) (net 6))
 (segment (start 170.91 94.61) (end 170.91 99.01) (width 0.25) (layer F.Cu) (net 6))
 (segment (start 170.91 99.01) (end 165.81 104.11) (width 0.25) (layer F.Cu) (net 6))
 (segment (start 174.05 89.31) (end 174.05 91.47) (width 0.25) (layer F.Cu) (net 6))
 (segment (start 165.81 104.11) (end 165.81 108.91) (width 0.25) (layer F.Cu) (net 6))
 (segment (start 165.81 108.91) (end 164.554 110.166) (width 0.25) (layer F.Cu) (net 6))
 (segment (start 174.05 85.65) (end 174.05 89.31) (width 0.25) (layer F.Cu) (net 6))
 (segment (start 170.11 81.71) (end 174.05 85.65) (width 0.25) (layer F.Cu) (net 6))
 (segment (start 162.101178 60.31) (end 162.101178 60.401178) (width 0.25) (layer F.Cu) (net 6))
 (segment (start 159.953089 58.161911) (end 162.101178 60.31) (width 0.25) (layer F.Cu) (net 6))
 (segment (start 164.91 63.21) (end 164.91 70.01) (width 0.25) (layer F.Cu) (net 6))
 (segment (start 162.101178 60.401178) (end 164.91 63.21) (width 0.25) (layer F.Cu) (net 6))
 (segment (start 164.91 70.01) (end 170.11 75.21) (width 0.25) (layer F.Cu) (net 6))
 (segment (start 170.11 75.21) (end 170.11 81.71) (width 0.25) (layer F.Cu) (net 6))
 (segment (start 93.91 111.31) (end 93.91 116.68275) (width 0.25) (layer F.Cu) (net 6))
 (segment (start 88.41 105.81) (end 93.91 111.31) (width 0.25) (layer F.Cu) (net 6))
 (segment (start 88.41 100.01) (end 88.41 105.81) (width 0.25) (layer F.Cu) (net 6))
 (segment (start 97.671125 120.443875) (end 94.073625 116.846375) (width 0.25) (layer F.Cu) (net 6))
 (segment (start 85.67 90.01) (end 85.67 91.16) (width 0.25) (layer F.Cu) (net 6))
 (segment (start 85.67 91.16) (end 85.61 91.22) (width 0.25) (layer F.Cu) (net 6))
 (segment (start 93.91 116.68275) (end 94.073625 116.846375) (width 0.25) (layer F.Cu) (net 6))
 (segment (start 85.61 91.22) (end 85.61 97.21) (width 0.25) (layer F.Cu) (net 6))
 (segment (start 85.61 97.21) (end 88.41 100.01) (width 0.25) (layer F.Cu) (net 6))
 (segment (start 85.67 79.45) (end 85.67 90.01) (width 0.25) (layer F.Cu) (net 6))
 (segment (start 90.11 75.01) (end 85.67 79.45) (width 0.25) (layer F.Cu) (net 6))
 (segment (start 90.11 70.01) (end 90.11 75.01) (width 0.25) (layer F.Cu) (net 6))
 (segment (start 96.964019 63.155981) (end 90.11 70.01) (width 0.25) (layer F.Cu) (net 6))
 (segment (start 97.671125 59.576125) (end 96.964019 60.283231) (width 0.25) (layer F.Cu) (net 6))
 (segment (start 96.964019 60.283231) (end 96.964019 63.155981) (width 0.25) (layer F.Cu) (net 6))
 (segment (start 102.906198 127.475) (end 96.773099 121.341901) (width 0.25) (layer F.Cu) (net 7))
 (segment (start 107.785 127.475) (end 102.906198 127.475) (width 0.25) (layer F.Cu) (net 7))
 (segment (start 130.01 135.349) (end 121.12 135.349) (width 0.25) (layer F.Cu) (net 7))
 (segment (start 113.373 133.063) (end 107.785 127.475) (width 0.25) (layer F.Cu) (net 7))
 (segment (start 118.834 133.063) (end 113.373 133.063) (width 0.25) (layer F.Cu) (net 7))
 (segment (start 121.12 135.349) (end 118.834 133.063) (width 0.25) (layer F.Cu) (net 7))
 (segment (start 137.884 135.349) (end 137.503 135.349) (width 0.25) (layer F.Cu) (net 7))
 (segment (start 137.503 135.349) (end 130.01 135.349) (width 0.25) (layer F.Cu) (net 7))
 (segment (start 129.01 135.349) (end 129.375 135.349) (width 0.25) (layer B.Cu) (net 7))
 (segment (start 127.673 135.349) (end 129.375 135.349) (width 0.25) (layer B.Cu) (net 7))
 (segment (start 126.19 133.866) (end 127.673 135.349) (width 0.25) (layer B.Cu) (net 7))
 (segment (start 126.19 127.91) (end 126.19 133.866) (width 0.25) (layer B.Cu) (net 7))
 (segment (start 146.774 127.348) (end 138.773 135.349) (width 0.25) (layer F.Cu) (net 7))
 (segment (start 156.607154 127.348) (end 146.774 127.348) (width 0.25) (layer F.Cu) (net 7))
 (segment (start 165.697 118.258154) (end 156.607154 127.348) (width 0.25) (layer F.Cu) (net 7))
 (segment (start 165.697 110.323) (end 165.697 118.258154) (width 0.25) (layer F.Cu) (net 7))
 (segment (start 166.91 109.11) (end 165.697 110.323) (width 0.25) (layer F.Cu) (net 7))
 (segment (start 175.32 91.095) (end 175.21 91.205) (width 0.25) (layer F.Cu) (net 7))
 (segment (start 166.91 104.81) (end 166.91 109.11) (width 0.25) (layer F.Cu) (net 7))
 (segment (start 175.21 91.205) (end 175.21 91.71) (width 0.25) (layer F.Cu) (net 7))
 (segment (start 175.21 91.71) (end 171.81 95.11) (width 0.25) (layer F.Cu) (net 7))
 (segment (start 138.773 135.349) (end 137.503 135.349) (width 0.25) (layer F.Cu) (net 7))
 (segment (start 175.32 89.945) (end 175.32 91.095) (width 0.25) (layer F.Cu) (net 7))
 (segment (start 171.81 95.11) (end 171.81 99.91) (width 0.25) (layer F.Cu) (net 7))
 (segment (start 171.81 99.91) (end 166.91 104.81) (width 0.25) (layer F.Cu) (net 7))
 (segment (start 84.4 90.525) (end 84.41 90.535) (width 0.25) (layer F.Cu) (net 7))
 (segment (start 84.4 89.375) (end 84.4 90.525) (width 0.25) (layer F.Cu) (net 7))
 (segment (start 84.41 90.535) (end 84.41 97.61) (width 0.25) (layer F.Cu) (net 7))
 (segment (start 84.41 97.61) (end 87.21 100.41) (width 0.25) (layer F.Cu) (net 7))
 (segment (start 87.21 100.41) (end 87.21 106.31) (width 0.25) (layer F.Cu) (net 7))
 (segment (start 91.925599 111.025599) (end 91.925599 116.494401) (width 0.25) (layer F.Cu) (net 7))
 (segment (start 87.21 106.31) (end 91.925599 111.025599) (width 0.25) (layer F.Cu) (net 7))
 (segment (start 96.773099 121.341901) (end 91.925599 116.494401) (width 0.25) (layer F.Cu) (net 7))
 (segment (start 175.32 85.52) (end 175.32 89.945) (width 0.25) (layer F.Cu) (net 7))
 (segment (start 171.31 74.21) (end 171.31 81.51) (width 0.25) (layer F.Cu) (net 7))
 (segment (start 166.11 69.01) (end 171.31 74.21) (width 0.25) (layer F.Cu) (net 7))
 (segment (start 156.13223 52.545) (end 166.11 62.52277) (width 0.25) (layer F.Cu) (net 7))
 (segment (start 148.171 52.545) (end 156.13223 52.545) (width 0.25) (layer F.Cu) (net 7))
 (segment (start 84.4 88.225) (end 84.81 87.815) (width 0.25) (layer F.Cu) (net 7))
 (segment (start 88.81 74.41) (end 88.81 69.81) (width 0.25) (layer F.Cu) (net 7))
 (segment (start 171.31 81.51) (end 175.32 85.52) (width 0.25) (layer F.Cu) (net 7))
 (segment (start 84.81 78.41) (end 88.81 74.41) (width 0.25) (layer F.Cu) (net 7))
 (segment (start 88.81 69.81) (end 94.958 63.662) (width 0.25) (layer F.Cu) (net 7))
 (segment (start 84.81 87.815) (end 84.81 78.41) (width 0.25) (layer F.Cu) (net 7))
 (segment (start 166.11 62.52277) (end 166.11 69.01) (width 0.25) (layer F.Cu) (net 7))
 (segment (start 112.992 48.354) (end 120.866 48.354) (width 0.25) (layer F.Cu) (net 7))
 (segment (start 84.4 89.375) (end 84.4 88.225) (width 0.25) (layer F.Cu) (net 7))
 (segment (start 124.549 44.671) (end 133.185 44.671) (width 0.25) (layer F.Cu) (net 7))
 (segment (start 94.958 63.662) (end 94.958 60.493198) (width 0.25) (layer F.Cu) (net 7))
 (segment (start 94.958 60.493198) (end 100.112198 55.339) (width 0.25) (layer F.Cu) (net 7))
 (segment (start 100.112198 55.339) (end 106.007 55.339) (width 0.25) (layer F.Cu) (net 7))
 (segment (start 120.866 48.354) (end 124.549 44.671) (width 0.25) (layer F.Cu) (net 7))
 (segment (start 106.007 55.339) (end 112.992 48.354) (width 0.25) (layer F.Cu) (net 7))
 (segment (start 133.185 44.671) (end 135.979 47.465) (width 0.25) (layer F.Cu) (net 7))
 (segment (start 135.979 47.465) (end 143.091 47.465) (width 0.25) (layer F.Cu) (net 7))
 (segment (start 143.091 47.465) (end 148.171 52.545) (width 0.25) (layer F.Cu) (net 7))
 (segment (start 132.55 79.35) (end 132.71 79.51) (width 0.25) (layer F.Cu) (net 1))
 (segment (start 132.55 64.955) (end 132.55 79.35) (width 0.25) (layer F.Cu) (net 1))
 (segment (start 114.071814 102.229084) (end 120.341916 102.229084) (width 0.25) (layer F.Cu) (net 1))
 (segment (start 126.753102 96.153102) (end 126.5855 95.9855) (width 0.25) (layer F.Cu) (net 1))
 (segment (start 132.55 96.153102) (end 126.753102 96.153102) (width 0.25) (layer F.Cu) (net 1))
 (segment (start 142.356084 105.959186) (end 132.55 96.153102) (width 0.25) (layer F.Cu) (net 1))
 (segment (start 120.341916 102.229084) (end 126.5855 95.9855) (width 0.25) (layer F.Cu) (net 1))
 (segment (start 126.5855 95.9855) (end 132.55 90.021) (width 0.25) (layer F.Cu) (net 1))
 (segment (start 132.71 89.861) (end 132.55 90.021) (width 0.25) (layer F.Cu) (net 1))
 (segment (start 132.71 79.51) (end 132.71 89.861) (width 0.25) (layer F.Cu) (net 1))
 (segment (start 129.320001 78.660001) (end 130.17 79.51) (width 0.25) (layer F.Cu) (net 2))
 (segment (start 129.110001 78.450001) (end 129.320001 78.660001) (width 0.25) (layer F.Cu) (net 2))
 (segment (start 129.110001 65.854999) (end 129.110001 78.450001) (width 0.25) (layer F.Cu) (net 2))
 (segment (start 130.01 64.955) (end 129.110001 65.854999) (width 0.25) (layer F.Cu) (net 2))
 (segment (start 145.11 105.121) (end 144.152135 104.163135) (width 0.25) (layer F.Cu) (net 2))
 (segment (start 145.11 106.31) (end 145.11 105.121) (width 0.25) (layer F.Cu) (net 2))
 (segment (start 143.51 107.91) (end 145.11 106.31) (width 0.25) (layer F.Cu) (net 2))
 (segment (start 141.31 107.91) (end 143.51 107.91) (width 0.25) (layer F.Cu) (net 2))
 (segment (start 115.867865 104.025135) (end 137.425135 104.025135) (width 0.25) (layer F.Cu) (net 2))
 (segment (start 137.425135 104.025135) (end 141.31 107.91) (width 0.25) (layer F.Cu) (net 2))
 (segment (start 144.152135 104.163135) (end 130.01 90.021) (width 0.25) (layer B.Cu) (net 2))
 (segment (start 130.17 89.861) (end 130.01 90.021) (width 0.25) (layer F.Cu) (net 2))
 (segment (start 130.17 79.51) (end 130.17 89.861) (width 0.25) (layer F.Cu) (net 2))
 (segment (start 126.780001 78.660001) (end 127.63 79.51) (width 0.25) (layer F.Cu) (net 3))
 (segment (start 126.570001 78.450001) (end 126.780001 78.660001) (width 0.25) (layer F.Cu) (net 3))
 (segment (start 126.570001 65.854999) (end 126.570001 78.450001) (width 0.25) (layer F.Cu) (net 3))
 (segment (start 127.47 64.955) (end 126.570001 65.854999) (width 0.25) (layer F.Cu) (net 3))
 (segment (start 118.563915 106.721185) (end 137.221185 106.721185) (width 0.25) (layer F.Cu) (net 3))
 (segment (start 117.663916 105.821186) (end 118.563915 106.721185) (width 0.25) (layer F.Cu) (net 3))
 (segment (start 137.221185 106.721185) (end 139.61 109.11) (width 0.25) (layer F.Cu) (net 3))
 (segment (start 139.61 109.11) (end 144.21 109.11) (width 0.25) (layer F.Cu) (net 3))
 (segment (start 145.948186 107.371814) (end 145.948186 106.971814) (width 0.25) (layer F.Cu) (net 3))
 (segment (start 144.21 109.11) (end 145.948186 107.371814) (width 0.25) (layer F.Cu) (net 3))
 (segment (start 145.948186 106.971814) (end 145.948186 102.367084) (width 0.25) (layer F.Cu) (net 3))
 (segment (start 116.391124 105.821186) (end 117.663916 105.821186) (width 0.25) (layer F.Cu) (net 3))
 (segment (start 127.47 90.021) (end 126.570001 90.920999) (width 0.25) (layer F.Cu) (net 3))
 (segment (start 126.570001 90.920999) (end 120.599001 90.920999) (width 0.25) (layer F.Cu) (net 3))
 (segment (start 115.021186 105.821186) (end 116.391124 105.821186) (width 0.25) (layer F.Cu) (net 3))
 (segment (start 127.63 89.861) (end 127.47 90.021) (width 0.25) (layer F.Cu) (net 3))
 (segment (start 127.63 79.51) (end 127.63 89.861) (width 0.25) (layer F.Cu) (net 3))
 (segment (start 112.31 103.11) (end 115.021186 105.821186) (width 0.25) (layer F.Cu) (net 3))
 (segment (start 112.31 99.21) (end 112.31 103.11) (width 0.25) (layer F.Cu) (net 3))
 (segment (start 120.599001 90.920999) (end 112.31 99.21) (width 0.25) (layer F.Cu) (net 3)))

